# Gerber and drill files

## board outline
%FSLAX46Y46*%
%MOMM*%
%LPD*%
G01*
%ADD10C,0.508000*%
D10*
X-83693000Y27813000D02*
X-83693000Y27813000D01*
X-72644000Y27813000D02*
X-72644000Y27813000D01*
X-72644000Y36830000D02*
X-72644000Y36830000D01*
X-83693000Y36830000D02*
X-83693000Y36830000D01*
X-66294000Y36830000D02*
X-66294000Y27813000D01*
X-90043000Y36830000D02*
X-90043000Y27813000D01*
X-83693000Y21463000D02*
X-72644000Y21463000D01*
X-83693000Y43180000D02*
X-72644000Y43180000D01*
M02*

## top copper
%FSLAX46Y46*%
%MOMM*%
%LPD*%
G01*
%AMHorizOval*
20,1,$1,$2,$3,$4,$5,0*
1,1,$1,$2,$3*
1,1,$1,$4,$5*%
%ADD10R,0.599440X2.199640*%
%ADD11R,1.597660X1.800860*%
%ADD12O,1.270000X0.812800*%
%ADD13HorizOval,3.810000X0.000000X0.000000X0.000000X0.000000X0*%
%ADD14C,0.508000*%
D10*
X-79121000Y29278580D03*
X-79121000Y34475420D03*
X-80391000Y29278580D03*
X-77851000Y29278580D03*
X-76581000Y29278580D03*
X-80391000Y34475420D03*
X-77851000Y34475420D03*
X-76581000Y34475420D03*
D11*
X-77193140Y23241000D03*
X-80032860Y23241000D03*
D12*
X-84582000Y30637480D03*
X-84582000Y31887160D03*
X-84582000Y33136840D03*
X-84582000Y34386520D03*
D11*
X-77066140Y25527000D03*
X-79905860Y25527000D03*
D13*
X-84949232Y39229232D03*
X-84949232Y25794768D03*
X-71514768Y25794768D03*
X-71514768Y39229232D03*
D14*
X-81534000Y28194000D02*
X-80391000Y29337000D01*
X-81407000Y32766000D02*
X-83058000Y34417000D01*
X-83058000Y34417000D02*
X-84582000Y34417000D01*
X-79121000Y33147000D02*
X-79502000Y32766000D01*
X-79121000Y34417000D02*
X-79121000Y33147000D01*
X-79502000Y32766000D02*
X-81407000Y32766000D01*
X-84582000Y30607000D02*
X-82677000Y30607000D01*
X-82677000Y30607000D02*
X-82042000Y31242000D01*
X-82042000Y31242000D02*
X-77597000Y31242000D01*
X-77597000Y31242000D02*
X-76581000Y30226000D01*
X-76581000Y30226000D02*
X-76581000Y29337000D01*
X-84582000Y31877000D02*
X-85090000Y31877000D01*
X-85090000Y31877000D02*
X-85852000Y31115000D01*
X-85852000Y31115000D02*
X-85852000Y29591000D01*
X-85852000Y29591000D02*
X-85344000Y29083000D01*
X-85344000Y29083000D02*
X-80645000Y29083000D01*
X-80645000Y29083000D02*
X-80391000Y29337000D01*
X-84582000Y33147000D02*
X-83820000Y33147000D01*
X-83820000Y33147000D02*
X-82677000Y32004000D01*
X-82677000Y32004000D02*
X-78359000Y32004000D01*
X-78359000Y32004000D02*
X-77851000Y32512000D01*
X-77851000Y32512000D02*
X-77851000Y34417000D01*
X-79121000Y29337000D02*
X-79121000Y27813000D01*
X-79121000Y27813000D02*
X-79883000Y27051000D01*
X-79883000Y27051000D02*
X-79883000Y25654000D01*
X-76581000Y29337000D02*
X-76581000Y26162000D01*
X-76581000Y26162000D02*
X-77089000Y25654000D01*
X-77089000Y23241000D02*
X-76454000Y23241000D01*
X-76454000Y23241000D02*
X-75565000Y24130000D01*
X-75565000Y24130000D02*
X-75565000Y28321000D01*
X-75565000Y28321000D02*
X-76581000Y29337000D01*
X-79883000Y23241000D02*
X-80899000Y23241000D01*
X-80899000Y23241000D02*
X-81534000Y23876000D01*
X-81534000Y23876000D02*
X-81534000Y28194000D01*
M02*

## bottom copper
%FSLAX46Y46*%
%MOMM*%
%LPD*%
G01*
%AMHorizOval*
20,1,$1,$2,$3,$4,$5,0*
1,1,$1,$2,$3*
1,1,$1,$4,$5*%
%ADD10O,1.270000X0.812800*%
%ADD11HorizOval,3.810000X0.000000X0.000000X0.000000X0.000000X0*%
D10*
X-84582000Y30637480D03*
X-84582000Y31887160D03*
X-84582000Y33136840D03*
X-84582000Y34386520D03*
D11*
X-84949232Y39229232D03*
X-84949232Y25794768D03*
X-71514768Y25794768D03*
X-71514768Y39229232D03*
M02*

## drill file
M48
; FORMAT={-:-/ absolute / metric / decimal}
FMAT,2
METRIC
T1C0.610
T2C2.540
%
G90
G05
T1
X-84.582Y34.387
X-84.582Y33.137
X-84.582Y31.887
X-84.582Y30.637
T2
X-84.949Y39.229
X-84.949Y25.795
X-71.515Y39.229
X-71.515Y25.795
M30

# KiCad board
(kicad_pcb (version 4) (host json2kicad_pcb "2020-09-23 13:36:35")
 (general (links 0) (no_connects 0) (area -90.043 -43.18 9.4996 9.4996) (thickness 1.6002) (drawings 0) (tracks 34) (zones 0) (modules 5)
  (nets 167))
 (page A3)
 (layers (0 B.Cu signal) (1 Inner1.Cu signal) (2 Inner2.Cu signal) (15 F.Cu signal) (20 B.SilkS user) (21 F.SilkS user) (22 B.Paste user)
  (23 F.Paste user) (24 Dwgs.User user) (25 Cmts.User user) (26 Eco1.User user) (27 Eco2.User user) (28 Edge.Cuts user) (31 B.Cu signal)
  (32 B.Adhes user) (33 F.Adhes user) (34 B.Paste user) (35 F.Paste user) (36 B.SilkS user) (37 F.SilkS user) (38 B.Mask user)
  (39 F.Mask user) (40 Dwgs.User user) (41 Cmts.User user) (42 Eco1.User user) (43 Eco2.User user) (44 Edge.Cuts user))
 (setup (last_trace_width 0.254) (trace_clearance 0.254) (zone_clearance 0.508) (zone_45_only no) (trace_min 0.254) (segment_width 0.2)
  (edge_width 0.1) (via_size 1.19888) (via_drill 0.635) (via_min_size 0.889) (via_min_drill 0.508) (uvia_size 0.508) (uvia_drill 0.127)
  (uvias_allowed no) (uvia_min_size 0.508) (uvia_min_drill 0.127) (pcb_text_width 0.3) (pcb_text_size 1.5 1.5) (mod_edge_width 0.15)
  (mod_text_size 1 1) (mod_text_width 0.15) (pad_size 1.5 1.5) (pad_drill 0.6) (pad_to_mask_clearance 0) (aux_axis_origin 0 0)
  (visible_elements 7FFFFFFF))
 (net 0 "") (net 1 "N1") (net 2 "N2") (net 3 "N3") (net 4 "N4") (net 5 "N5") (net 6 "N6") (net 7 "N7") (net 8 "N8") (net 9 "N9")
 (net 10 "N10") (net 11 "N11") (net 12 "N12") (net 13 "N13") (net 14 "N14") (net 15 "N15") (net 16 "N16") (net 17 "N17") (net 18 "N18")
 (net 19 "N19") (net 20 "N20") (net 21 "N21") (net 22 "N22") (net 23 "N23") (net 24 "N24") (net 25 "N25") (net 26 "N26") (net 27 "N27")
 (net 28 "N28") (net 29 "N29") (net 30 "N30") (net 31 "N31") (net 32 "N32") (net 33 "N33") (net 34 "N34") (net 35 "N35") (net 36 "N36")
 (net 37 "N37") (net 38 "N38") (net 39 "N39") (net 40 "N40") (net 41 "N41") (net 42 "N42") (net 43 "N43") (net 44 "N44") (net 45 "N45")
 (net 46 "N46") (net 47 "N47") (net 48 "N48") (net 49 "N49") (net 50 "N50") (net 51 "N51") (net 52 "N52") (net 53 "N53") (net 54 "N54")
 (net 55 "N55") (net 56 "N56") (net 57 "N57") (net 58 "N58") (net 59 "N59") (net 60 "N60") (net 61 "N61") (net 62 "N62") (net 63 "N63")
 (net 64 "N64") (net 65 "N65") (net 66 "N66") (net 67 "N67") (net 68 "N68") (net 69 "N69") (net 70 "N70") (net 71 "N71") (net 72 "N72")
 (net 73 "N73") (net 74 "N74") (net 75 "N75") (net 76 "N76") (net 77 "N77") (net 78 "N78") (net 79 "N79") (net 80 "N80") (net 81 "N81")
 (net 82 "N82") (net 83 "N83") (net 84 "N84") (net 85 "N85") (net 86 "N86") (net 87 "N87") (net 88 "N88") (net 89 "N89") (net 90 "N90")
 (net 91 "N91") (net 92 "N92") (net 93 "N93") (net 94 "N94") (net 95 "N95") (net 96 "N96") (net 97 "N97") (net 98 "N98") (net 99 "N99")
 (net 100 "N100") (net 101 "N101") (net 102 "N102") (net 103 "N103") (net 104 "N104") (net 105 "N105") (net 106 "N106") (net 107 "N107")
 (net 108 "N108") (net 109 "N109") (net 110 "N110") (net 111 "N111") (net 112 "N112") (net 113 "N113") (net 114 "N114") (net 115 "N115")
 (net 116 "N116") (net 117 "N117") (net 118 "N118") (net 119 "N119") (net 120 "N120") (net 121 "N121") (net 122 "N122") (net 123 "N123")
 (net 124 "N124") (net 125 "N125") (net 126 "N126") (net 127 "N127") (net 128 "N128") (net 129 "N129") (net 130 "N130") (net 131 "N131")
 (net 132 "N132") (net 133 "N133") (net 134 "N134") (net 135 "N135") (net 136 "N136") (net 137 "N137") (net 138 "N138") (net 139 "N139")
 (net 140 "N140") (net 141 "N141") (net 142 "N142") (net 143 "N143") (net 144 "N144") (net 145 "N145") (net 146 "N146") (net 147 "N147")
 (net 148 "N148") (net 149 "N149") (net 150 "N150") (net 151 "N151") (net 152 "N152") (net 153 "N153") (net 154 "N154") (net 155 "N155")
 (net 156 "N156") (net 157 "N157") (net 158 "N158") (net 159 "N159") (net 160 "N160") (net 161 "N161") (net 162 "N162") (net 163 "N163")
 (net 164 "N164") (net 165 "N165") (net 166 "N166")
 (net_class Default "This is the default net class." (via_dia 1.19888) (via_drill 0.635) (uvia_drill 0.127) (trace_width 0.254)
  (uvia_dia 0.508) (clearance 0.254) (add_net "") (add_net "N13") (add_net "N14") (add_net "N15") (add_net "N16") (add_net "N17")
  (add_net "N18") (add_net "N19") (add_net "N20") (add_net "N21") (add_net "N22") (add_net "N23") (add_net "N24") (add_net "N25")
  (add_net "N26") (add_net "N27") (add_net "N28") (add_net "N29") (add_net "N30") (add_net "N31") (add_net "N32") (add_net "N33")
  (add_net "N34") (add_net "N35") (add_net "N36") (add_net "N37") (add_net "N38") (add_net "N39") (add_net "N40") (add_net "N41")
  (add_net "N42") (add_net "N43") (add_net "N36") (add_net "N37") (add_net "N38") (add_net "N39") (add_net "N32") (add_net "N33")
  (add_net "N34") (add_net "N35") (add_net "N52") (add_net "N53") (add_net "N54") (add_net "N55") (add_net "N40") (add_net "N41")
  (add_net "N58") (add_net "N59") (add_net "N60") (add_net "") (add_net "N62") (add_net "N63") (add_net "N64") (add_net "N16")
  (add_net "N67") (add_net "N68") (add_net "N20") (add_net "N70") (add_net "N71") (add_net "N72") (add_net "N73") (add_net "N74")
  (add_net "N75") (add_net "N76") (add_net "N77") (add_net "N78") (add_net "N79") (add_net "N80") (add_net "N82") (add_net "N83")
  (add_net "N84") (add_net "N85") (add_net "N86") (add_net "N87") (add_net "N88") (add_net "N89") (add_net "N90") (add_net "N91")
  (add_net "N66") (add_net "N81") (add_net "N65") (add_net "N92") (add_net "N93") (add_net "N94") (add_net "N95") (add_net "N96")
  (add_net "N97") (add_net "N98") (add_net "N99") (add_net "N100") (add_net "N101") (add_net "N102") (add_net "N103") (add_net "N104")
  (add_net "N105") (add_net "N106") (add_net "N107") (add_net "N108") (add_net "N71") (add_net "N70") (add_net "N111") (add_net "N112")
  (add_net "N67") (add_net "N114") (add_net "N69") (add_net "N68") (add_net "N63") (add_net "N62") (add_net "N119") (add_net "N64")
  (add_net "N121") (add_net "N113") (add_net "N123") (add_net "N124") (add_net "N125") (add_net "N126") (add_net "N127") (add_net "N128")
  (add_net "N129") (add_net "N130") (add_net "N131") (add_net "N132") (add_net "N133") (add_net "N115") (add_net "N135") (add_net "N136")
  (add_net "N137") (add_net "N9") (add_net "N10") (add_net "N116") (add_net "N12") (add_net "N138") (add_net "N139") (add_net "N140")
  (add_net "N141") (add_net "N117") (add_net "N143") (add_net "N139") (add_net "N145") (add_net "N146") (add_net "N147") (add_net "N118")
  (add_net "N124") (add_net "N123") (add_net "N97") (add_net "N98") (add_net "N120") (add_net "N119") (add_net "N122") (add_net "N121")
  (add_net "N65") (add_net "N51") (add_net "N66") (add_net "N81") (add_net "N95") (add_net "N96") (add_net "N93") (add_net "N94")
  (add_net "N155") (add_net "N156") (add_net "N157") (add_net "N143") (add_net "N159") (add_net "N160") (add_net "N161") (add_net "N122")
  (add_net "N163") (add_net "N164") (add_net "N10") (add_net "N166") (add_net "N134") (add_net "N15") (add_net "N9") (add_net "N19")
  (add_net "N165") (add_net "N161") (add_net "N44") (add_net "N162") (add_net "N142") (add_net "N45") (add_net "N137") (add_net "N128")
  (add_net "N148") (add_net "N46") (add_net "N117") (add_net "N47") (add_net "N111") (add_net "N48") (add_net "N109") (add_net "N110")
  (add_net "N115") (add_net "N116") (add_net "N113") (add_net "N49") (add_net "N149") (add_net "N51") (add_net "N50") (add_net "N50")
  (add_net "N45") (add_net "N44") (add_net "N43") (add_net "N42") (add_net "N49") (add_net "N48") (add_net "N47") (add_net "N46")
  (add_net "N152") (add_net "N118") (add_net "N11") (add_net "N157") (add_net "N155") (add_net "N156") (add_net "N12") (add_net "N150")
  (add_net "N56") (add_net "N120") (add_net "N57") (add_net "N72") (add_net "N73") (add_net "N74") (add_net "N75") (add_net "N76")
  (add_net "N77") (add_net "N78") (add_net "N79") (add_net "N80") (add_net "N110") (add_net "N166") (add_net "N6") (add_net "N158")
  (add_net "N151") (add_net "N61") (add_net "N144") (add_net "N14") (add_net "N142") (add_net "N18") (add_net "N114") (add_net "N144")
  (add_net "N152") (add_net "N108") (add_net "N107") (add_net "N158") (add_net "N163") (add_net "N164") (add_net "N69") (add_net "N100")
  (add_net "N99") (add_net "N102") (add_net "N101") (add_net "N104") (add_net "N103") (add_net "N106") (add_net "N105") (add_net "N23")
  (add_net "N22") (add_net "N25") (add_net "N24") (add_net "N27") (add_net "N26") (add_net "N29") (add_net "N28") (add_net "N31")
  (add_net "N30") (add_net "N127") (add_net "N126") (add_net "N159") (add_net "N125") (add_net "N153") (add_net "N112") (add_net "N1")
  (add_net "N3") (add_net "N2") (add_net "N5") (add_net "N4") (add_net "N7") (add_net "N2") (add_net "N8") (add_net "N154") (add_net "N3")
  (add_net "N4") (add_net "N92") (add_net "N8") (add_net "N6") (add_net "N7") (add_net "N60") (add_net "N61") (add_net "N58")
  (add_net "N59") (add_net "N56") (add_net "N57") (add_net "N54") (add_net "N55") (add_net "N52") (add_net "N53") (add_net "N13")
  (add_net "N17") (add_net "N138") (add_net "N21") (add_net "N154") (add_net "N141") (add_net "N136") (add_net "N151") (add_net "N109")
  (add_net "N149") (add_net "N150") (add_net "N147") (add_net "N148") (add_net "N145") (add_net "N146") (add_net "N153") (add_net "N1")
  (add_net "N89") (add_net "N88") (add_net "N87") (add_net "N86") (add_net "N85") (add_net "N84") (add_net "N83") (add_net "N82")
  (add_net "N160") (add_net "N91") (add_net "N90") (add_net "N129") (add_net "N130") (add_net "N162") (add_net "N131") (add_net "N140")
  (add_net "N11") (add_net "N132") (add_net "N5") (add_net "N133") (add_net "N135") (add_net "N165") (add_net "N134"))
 (gr_line (start -83.693 -27.813) (end -83.693 -27.813) (angle -90.00) (width 0.508) (layer Edge.Cuts))
 (gr_line (start -72.644 -27.813) (end -72.644 -27.813) (angle -90.00) (width 0.508) (layer Edge.Cuts))
 (gr_line (start -72.644 -36.83) (end -72.644 -36.83) (angle -90.00) (width 0.508) (layer Edge.Cuts))
 (gr_line (start -83.693 -36.83) (end -83.693 -36.83) (angle -90.00) (width 0.508) (layer Edge.Cuts))
 (gr_line (start -66.294 -36.83) (end -66.294 -27.813) (angle 51566.20) (width 0.508) (layer Edge.Cuts))
 (gr_line (start -90.043 -36.83) (end -90.043 -27.813) (angle 51566.20) (width 0.508) (layer Edge.Cuts))
 (gr_line (start -83.693 -21.463) (end -72.644 -21.463) (angle 51566.20) (width 0.508) (layer Edge.Cuts))
 (gr_line (start -83.693 -43.18) (end -72.644 -43.18) (angle 51566.20) (width 0.508) (layer Edge.Cuts))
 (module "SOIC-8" (layer "F.Cu") (at -78.486 -31.877 0.00)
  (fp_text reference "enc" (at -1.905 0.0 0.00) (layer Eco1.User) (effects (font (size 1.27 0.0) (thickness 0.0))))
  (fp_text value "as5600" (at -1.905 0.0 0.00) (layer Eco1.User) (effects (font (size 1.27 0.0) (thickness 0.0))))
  (pad 2 smd rect (at -0.635 2.59842 0.00) (size 0.59944 2.19964) (drill 0.0) (layers "F.Cu" "F.Paste") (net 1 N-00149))
  (pad 7 smd rect (at -0.635 -2.59842 0.00) (size 0.59944 2.19964) (drill 0.0) (layers "F.Cu" "F.Paste") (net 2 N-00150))
  (pad 1 smd rect (at -1.905 2.59842 0.00) (size 0.59944 2.19964) (drill 0.0) (layers "F.Cu" "F.Paste") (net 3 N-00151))
  (pad 3 smd rect (at 0.635 2.59842 0.00) (size 0.59944 2.19964) (drill 0.0) (layers "F.Cu" "F.Paste") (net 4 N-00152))
  (pad 4 smd rect (at 1.905 2.59842 0.00) (size 0.59944 2.19964) (drill 0.0) (layers "F.Cu" "F.Paste") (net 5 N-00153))
  (pad 8 smd rect (at -1.905 -2.59842 0.00) (size 0.59944 2.19964) (drill 0.0) (layers "F.Cu" "F.Paste") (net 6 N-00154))
  (pad 6 smd rect (at 0.635 -2.59842 0.00) (size 0.59944 2.19964) (drill 0.0) (layers "F.Cu" "F.Paste") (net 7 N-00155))
  (pad 5 smd rect (at 1.905 -2.59842 0.00) (size 0.59944 2.19964) (drill 0.0) (layers "F.Cu" "F.Paste") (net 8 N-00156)))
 (segment (start -81.534 -28.194) (end -80.391 -29.337) (width 0.508) (layer F.Cu) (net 3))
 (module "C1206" (layer "F.Cu") (at -78.613 -23.241 0.00)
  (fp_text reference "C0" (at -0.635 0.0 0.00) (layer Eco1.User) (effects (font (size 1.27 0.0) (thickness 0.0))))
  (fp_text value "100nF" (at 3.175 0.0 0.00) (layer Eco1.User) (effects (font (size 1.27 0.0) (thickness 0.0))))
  (pad 2 smd rect (at 1.41986 0.0 0.00) (size 1.59766 1.80086) (drill 0.0) (layers "F.Cu" "F.Paste") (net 5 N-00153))
  (pad 1 smd rect (at -1.41986 0.0 0.00) (size 1.59766 1.80086) (drill 0.0) (layers "F.Cu" "F.Paste") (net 3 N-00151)))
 (segment (start -81.407 -32.766) (end -83.058 -34.417) (width 0.508) (layer F.Cu) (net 2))
 (segment (start -83.058 -34.417) (end -84.582 -34.417) (width 0.508) (layer F.Cu) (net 2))
 (segment (start -79.121 -33.147) (end -79.502 -32.766) (width 0.508) (layer F.Cu) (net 2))
 (segment (start -79.121 -34.417) (end -79.121 -33.147) (width 0.508) (layer F.Cu) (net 2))
 (segment (start -79.502 -32.766) (end -81.407 -32.766) (width 0.508) (layer F.Cu) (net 2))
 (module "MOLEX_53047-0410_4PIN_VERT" (layer "F.Cu") (at -84.582 -32.512 90.00)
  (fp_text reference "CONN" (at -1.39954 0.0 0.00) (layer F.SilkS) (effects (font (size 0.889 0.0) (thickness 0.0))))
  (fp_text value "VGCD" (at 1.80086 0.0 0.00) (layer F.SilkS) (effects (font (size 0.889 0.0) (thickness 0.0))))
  (pad 1 thru_hole oval (at -1.87452 0.0 90.00) (size 0.8128 1.27) (drill 0.6096)
   (layers "B.Cu" "Inner1.Cu" "Inner2.Cu" "F.Cu" "F.SilkS" "B.Paste" "F.Paste") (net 5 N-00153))
  (pad 2 thru_hole oval (at -0.62484 0.0 90.00) (size 0.8128 1.27) (drill 0.6096)
   (layers "B.Cu" "Inner1.Cu" "Inner2.Cu" "F.Cu" "F.SilkS" "B.Paste" "F.Paste") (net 3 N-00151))
  (pad 3 thru_hole oval (at 0.62484 0.0 90.00) (size 0.8128 1.27) (drill 0.6096)
   (layers "B.Cu" "Inner1.Cu" "Inner2.Cu" "F.Cu" "F.SilkS" "B.Paste" "F.Paste") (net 7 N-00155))
  (pad 4 thru_hole oval (at 1.87452 0.0 90.00) (size 0.8128 1.27) (drill 0.6096)
   (layers "B.Cu" "Inner1.Cu" "Inner2.Cu" "F.Cu" "F.SilkS" "B.Paste" "F.Paste") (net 2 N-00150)))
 (segment (start -84.582 -30.607) (end -82.677 -30.607) (width 0.508) (layer F.Cu) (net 5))
 (segment (start -82.677 -30.607) (end -82.042 -31.242) (width 0.508) (layer F.Cu) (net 5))
 (segment (start -82.042 -31.242) (end -77.597 -31.242) (width 0.508) (layer F.Cu) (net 5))
 (segment (start -77.597 -31.242) (end -76.581 -30.226) (width 0.508) (layer F.Cu) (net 5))
 (segment (start -76.581 -30.226) (end -76.581 -29.337) (width 0.508) (layer F.Cu) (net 5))
 (segment (start -84.582 -31.877) (end -85.09 -31.877) (width 0.508) (layer F.Cu) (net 3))
 (segment (start -85.09 -31.877) (end -85.852 -31.115) (width 0.508) (layer F.Cu) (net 3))
 (segment (start -85.852 -31.115) (end -85.852 -29.591) (width 0.508) (layer F.Cu) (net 3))
 (segment (start -85.852 -29.591) (end -85.344 -29.083) (width 0.508) (layer F.Cu) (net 3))
 (segment (start -85.344 -29.083) (end -80.645 -29.083) (width 0.508) (layer F.Cu) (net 3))
 (segment (start -80.645 -29.083) (end -80.391 -29.337) (width 0.508) (layer F.Cu) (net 3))
 (segment (start -84.582 -33.147) (end -83.82 -33.147) (width 0.508) (layer F.Cu) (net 7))
 (segment (start -83.82 -33.147) (end -82.677 -32.004) (width 0.508) (layer F.Cu) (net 7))
 (segment (start -82.677 -32.004) (end -78.359 -32.004) (width 0.508) (layer F.Cu) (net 7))
 (segment (start -78.359 -32.004) (end -77.851 -32.512) (width 0.508) (layer F.Cu) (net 7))
 (segment (start -77.851 -32.512) (end -77.851 -34.417) (width 0.508) (layer F.Cu) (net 7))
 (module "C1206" (layer "F.Cu") (at -78.486 -25.527 0.00)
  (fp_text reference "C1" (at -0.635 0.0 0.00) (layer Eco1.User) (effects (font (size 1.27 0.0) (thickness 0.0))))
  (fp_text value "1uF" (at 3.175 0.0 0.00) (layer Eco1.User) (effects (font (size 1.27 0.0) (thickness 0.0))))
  (pad 2 smd rect (at 1.41986 0.0 0.00) (size 1.59766 1.80086) (drill 0.0) (layers "F.Cu" "F.Paste") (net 5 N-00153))
  (pad 1 smd rect (at -1.41986 0.0 0.00) (size 1.59766 1.80086) (drill 0.0) (layers "F.Cu" "F.Paste") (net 1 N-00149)))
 (segment (start -79.121 -29.337) (end -79.121 -27.813) (width 0.508) (layer F.Cu) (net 1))
 (segment (start -79.121 -27.813) (end -79.883 -27.051) (width 0.508) (layer F.Cu) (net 1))
 (segment (start -79.883 -27.051) (end -79.883 -25.654) (width 0.508) (layer F.Cu) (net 1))
 (segment (start -76.581 -29.337) (end -76.581 -26.162) (width 0.508) (layer F.Cu) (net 5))
 (segment (start -76.581 -26.162) (end -77.089 -25.654) (width 0.508) (layer F.Cu) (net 5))
 (segment (start -77.089 -23.241) (end -76.454 -23.241) (width 0.508) (layer F.Cu) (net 5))
 (segment (start -76.454 -23.241) (end -75.565 -24.13) (width 0.508) (layer F.Cu) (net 5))
 (segment (start -75.565 -24.13) (end -75.565 -28.321) (width 0.508) (layer F.Cu) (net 5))
 (segment (start -75.565 -28.321) (end -76.581 -29.337) (width 0.508) (layer F.Cu) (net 5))
 (segment (start -79.883 -23.241) (end -80.899 -23.241) (width 0.508) (layer F.Cu) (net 3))
 (segment (start -80.899 -23.241) (end -81.534 -23.876) (width 0.508) (layer F.Cu) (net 3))
 (segment (start -81.534 -23.876) (end -81.534 -28.194) (width 0.508) (layer F.Cu) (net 3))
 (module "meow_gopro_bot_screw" (layer "F.Cu") (at -78.232 -32.512 -135.00)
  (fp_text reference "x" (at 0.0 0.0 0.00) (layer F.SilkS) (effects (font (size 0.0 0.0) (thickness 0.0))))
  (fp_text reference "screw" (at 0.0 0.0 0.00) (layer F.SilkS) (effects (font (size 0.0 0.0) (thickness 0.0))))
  (pad S0 thru_hole oval (at 0.0 9.4996 -135.00) (size 3.81 3.81) (drill 2.54)
   (layers "B.Cu" "Inner1.Cu" "Inner2.Cu" "F.Cu" "B.Paste" "F.Paste") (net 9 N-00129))
  (pad S1 thru_hole oval (at 9.4996 0.0 -135.00) (size 3.81 3.81) (drill 2.54)
   (layers "B.Cu" "Inner1.Cu" "Inner2.Cu" "F.Cu" "B.Paste" "F.Paste") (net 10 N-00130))
  (pad S2 thru_hole oval (at 0.0 -9.4996 -135.00) (size 3.81 3.81) (drill 2.54)
   (layers "B.Cu" "Inner1.Cu" "Inner2.Cu" "F.Cu" "B.Paste" "F.Paste") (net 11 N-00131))
  (pad S3 thru_hole oval (at -9.4996 0.0 -135.00) (size 3.81 3.81) (drill 2.54)
   (layers "B.Cu" "Inner1.Cu" "Inner2.Cu" "F.Cu" "B.Paste" "F.Paste") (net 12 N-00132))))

